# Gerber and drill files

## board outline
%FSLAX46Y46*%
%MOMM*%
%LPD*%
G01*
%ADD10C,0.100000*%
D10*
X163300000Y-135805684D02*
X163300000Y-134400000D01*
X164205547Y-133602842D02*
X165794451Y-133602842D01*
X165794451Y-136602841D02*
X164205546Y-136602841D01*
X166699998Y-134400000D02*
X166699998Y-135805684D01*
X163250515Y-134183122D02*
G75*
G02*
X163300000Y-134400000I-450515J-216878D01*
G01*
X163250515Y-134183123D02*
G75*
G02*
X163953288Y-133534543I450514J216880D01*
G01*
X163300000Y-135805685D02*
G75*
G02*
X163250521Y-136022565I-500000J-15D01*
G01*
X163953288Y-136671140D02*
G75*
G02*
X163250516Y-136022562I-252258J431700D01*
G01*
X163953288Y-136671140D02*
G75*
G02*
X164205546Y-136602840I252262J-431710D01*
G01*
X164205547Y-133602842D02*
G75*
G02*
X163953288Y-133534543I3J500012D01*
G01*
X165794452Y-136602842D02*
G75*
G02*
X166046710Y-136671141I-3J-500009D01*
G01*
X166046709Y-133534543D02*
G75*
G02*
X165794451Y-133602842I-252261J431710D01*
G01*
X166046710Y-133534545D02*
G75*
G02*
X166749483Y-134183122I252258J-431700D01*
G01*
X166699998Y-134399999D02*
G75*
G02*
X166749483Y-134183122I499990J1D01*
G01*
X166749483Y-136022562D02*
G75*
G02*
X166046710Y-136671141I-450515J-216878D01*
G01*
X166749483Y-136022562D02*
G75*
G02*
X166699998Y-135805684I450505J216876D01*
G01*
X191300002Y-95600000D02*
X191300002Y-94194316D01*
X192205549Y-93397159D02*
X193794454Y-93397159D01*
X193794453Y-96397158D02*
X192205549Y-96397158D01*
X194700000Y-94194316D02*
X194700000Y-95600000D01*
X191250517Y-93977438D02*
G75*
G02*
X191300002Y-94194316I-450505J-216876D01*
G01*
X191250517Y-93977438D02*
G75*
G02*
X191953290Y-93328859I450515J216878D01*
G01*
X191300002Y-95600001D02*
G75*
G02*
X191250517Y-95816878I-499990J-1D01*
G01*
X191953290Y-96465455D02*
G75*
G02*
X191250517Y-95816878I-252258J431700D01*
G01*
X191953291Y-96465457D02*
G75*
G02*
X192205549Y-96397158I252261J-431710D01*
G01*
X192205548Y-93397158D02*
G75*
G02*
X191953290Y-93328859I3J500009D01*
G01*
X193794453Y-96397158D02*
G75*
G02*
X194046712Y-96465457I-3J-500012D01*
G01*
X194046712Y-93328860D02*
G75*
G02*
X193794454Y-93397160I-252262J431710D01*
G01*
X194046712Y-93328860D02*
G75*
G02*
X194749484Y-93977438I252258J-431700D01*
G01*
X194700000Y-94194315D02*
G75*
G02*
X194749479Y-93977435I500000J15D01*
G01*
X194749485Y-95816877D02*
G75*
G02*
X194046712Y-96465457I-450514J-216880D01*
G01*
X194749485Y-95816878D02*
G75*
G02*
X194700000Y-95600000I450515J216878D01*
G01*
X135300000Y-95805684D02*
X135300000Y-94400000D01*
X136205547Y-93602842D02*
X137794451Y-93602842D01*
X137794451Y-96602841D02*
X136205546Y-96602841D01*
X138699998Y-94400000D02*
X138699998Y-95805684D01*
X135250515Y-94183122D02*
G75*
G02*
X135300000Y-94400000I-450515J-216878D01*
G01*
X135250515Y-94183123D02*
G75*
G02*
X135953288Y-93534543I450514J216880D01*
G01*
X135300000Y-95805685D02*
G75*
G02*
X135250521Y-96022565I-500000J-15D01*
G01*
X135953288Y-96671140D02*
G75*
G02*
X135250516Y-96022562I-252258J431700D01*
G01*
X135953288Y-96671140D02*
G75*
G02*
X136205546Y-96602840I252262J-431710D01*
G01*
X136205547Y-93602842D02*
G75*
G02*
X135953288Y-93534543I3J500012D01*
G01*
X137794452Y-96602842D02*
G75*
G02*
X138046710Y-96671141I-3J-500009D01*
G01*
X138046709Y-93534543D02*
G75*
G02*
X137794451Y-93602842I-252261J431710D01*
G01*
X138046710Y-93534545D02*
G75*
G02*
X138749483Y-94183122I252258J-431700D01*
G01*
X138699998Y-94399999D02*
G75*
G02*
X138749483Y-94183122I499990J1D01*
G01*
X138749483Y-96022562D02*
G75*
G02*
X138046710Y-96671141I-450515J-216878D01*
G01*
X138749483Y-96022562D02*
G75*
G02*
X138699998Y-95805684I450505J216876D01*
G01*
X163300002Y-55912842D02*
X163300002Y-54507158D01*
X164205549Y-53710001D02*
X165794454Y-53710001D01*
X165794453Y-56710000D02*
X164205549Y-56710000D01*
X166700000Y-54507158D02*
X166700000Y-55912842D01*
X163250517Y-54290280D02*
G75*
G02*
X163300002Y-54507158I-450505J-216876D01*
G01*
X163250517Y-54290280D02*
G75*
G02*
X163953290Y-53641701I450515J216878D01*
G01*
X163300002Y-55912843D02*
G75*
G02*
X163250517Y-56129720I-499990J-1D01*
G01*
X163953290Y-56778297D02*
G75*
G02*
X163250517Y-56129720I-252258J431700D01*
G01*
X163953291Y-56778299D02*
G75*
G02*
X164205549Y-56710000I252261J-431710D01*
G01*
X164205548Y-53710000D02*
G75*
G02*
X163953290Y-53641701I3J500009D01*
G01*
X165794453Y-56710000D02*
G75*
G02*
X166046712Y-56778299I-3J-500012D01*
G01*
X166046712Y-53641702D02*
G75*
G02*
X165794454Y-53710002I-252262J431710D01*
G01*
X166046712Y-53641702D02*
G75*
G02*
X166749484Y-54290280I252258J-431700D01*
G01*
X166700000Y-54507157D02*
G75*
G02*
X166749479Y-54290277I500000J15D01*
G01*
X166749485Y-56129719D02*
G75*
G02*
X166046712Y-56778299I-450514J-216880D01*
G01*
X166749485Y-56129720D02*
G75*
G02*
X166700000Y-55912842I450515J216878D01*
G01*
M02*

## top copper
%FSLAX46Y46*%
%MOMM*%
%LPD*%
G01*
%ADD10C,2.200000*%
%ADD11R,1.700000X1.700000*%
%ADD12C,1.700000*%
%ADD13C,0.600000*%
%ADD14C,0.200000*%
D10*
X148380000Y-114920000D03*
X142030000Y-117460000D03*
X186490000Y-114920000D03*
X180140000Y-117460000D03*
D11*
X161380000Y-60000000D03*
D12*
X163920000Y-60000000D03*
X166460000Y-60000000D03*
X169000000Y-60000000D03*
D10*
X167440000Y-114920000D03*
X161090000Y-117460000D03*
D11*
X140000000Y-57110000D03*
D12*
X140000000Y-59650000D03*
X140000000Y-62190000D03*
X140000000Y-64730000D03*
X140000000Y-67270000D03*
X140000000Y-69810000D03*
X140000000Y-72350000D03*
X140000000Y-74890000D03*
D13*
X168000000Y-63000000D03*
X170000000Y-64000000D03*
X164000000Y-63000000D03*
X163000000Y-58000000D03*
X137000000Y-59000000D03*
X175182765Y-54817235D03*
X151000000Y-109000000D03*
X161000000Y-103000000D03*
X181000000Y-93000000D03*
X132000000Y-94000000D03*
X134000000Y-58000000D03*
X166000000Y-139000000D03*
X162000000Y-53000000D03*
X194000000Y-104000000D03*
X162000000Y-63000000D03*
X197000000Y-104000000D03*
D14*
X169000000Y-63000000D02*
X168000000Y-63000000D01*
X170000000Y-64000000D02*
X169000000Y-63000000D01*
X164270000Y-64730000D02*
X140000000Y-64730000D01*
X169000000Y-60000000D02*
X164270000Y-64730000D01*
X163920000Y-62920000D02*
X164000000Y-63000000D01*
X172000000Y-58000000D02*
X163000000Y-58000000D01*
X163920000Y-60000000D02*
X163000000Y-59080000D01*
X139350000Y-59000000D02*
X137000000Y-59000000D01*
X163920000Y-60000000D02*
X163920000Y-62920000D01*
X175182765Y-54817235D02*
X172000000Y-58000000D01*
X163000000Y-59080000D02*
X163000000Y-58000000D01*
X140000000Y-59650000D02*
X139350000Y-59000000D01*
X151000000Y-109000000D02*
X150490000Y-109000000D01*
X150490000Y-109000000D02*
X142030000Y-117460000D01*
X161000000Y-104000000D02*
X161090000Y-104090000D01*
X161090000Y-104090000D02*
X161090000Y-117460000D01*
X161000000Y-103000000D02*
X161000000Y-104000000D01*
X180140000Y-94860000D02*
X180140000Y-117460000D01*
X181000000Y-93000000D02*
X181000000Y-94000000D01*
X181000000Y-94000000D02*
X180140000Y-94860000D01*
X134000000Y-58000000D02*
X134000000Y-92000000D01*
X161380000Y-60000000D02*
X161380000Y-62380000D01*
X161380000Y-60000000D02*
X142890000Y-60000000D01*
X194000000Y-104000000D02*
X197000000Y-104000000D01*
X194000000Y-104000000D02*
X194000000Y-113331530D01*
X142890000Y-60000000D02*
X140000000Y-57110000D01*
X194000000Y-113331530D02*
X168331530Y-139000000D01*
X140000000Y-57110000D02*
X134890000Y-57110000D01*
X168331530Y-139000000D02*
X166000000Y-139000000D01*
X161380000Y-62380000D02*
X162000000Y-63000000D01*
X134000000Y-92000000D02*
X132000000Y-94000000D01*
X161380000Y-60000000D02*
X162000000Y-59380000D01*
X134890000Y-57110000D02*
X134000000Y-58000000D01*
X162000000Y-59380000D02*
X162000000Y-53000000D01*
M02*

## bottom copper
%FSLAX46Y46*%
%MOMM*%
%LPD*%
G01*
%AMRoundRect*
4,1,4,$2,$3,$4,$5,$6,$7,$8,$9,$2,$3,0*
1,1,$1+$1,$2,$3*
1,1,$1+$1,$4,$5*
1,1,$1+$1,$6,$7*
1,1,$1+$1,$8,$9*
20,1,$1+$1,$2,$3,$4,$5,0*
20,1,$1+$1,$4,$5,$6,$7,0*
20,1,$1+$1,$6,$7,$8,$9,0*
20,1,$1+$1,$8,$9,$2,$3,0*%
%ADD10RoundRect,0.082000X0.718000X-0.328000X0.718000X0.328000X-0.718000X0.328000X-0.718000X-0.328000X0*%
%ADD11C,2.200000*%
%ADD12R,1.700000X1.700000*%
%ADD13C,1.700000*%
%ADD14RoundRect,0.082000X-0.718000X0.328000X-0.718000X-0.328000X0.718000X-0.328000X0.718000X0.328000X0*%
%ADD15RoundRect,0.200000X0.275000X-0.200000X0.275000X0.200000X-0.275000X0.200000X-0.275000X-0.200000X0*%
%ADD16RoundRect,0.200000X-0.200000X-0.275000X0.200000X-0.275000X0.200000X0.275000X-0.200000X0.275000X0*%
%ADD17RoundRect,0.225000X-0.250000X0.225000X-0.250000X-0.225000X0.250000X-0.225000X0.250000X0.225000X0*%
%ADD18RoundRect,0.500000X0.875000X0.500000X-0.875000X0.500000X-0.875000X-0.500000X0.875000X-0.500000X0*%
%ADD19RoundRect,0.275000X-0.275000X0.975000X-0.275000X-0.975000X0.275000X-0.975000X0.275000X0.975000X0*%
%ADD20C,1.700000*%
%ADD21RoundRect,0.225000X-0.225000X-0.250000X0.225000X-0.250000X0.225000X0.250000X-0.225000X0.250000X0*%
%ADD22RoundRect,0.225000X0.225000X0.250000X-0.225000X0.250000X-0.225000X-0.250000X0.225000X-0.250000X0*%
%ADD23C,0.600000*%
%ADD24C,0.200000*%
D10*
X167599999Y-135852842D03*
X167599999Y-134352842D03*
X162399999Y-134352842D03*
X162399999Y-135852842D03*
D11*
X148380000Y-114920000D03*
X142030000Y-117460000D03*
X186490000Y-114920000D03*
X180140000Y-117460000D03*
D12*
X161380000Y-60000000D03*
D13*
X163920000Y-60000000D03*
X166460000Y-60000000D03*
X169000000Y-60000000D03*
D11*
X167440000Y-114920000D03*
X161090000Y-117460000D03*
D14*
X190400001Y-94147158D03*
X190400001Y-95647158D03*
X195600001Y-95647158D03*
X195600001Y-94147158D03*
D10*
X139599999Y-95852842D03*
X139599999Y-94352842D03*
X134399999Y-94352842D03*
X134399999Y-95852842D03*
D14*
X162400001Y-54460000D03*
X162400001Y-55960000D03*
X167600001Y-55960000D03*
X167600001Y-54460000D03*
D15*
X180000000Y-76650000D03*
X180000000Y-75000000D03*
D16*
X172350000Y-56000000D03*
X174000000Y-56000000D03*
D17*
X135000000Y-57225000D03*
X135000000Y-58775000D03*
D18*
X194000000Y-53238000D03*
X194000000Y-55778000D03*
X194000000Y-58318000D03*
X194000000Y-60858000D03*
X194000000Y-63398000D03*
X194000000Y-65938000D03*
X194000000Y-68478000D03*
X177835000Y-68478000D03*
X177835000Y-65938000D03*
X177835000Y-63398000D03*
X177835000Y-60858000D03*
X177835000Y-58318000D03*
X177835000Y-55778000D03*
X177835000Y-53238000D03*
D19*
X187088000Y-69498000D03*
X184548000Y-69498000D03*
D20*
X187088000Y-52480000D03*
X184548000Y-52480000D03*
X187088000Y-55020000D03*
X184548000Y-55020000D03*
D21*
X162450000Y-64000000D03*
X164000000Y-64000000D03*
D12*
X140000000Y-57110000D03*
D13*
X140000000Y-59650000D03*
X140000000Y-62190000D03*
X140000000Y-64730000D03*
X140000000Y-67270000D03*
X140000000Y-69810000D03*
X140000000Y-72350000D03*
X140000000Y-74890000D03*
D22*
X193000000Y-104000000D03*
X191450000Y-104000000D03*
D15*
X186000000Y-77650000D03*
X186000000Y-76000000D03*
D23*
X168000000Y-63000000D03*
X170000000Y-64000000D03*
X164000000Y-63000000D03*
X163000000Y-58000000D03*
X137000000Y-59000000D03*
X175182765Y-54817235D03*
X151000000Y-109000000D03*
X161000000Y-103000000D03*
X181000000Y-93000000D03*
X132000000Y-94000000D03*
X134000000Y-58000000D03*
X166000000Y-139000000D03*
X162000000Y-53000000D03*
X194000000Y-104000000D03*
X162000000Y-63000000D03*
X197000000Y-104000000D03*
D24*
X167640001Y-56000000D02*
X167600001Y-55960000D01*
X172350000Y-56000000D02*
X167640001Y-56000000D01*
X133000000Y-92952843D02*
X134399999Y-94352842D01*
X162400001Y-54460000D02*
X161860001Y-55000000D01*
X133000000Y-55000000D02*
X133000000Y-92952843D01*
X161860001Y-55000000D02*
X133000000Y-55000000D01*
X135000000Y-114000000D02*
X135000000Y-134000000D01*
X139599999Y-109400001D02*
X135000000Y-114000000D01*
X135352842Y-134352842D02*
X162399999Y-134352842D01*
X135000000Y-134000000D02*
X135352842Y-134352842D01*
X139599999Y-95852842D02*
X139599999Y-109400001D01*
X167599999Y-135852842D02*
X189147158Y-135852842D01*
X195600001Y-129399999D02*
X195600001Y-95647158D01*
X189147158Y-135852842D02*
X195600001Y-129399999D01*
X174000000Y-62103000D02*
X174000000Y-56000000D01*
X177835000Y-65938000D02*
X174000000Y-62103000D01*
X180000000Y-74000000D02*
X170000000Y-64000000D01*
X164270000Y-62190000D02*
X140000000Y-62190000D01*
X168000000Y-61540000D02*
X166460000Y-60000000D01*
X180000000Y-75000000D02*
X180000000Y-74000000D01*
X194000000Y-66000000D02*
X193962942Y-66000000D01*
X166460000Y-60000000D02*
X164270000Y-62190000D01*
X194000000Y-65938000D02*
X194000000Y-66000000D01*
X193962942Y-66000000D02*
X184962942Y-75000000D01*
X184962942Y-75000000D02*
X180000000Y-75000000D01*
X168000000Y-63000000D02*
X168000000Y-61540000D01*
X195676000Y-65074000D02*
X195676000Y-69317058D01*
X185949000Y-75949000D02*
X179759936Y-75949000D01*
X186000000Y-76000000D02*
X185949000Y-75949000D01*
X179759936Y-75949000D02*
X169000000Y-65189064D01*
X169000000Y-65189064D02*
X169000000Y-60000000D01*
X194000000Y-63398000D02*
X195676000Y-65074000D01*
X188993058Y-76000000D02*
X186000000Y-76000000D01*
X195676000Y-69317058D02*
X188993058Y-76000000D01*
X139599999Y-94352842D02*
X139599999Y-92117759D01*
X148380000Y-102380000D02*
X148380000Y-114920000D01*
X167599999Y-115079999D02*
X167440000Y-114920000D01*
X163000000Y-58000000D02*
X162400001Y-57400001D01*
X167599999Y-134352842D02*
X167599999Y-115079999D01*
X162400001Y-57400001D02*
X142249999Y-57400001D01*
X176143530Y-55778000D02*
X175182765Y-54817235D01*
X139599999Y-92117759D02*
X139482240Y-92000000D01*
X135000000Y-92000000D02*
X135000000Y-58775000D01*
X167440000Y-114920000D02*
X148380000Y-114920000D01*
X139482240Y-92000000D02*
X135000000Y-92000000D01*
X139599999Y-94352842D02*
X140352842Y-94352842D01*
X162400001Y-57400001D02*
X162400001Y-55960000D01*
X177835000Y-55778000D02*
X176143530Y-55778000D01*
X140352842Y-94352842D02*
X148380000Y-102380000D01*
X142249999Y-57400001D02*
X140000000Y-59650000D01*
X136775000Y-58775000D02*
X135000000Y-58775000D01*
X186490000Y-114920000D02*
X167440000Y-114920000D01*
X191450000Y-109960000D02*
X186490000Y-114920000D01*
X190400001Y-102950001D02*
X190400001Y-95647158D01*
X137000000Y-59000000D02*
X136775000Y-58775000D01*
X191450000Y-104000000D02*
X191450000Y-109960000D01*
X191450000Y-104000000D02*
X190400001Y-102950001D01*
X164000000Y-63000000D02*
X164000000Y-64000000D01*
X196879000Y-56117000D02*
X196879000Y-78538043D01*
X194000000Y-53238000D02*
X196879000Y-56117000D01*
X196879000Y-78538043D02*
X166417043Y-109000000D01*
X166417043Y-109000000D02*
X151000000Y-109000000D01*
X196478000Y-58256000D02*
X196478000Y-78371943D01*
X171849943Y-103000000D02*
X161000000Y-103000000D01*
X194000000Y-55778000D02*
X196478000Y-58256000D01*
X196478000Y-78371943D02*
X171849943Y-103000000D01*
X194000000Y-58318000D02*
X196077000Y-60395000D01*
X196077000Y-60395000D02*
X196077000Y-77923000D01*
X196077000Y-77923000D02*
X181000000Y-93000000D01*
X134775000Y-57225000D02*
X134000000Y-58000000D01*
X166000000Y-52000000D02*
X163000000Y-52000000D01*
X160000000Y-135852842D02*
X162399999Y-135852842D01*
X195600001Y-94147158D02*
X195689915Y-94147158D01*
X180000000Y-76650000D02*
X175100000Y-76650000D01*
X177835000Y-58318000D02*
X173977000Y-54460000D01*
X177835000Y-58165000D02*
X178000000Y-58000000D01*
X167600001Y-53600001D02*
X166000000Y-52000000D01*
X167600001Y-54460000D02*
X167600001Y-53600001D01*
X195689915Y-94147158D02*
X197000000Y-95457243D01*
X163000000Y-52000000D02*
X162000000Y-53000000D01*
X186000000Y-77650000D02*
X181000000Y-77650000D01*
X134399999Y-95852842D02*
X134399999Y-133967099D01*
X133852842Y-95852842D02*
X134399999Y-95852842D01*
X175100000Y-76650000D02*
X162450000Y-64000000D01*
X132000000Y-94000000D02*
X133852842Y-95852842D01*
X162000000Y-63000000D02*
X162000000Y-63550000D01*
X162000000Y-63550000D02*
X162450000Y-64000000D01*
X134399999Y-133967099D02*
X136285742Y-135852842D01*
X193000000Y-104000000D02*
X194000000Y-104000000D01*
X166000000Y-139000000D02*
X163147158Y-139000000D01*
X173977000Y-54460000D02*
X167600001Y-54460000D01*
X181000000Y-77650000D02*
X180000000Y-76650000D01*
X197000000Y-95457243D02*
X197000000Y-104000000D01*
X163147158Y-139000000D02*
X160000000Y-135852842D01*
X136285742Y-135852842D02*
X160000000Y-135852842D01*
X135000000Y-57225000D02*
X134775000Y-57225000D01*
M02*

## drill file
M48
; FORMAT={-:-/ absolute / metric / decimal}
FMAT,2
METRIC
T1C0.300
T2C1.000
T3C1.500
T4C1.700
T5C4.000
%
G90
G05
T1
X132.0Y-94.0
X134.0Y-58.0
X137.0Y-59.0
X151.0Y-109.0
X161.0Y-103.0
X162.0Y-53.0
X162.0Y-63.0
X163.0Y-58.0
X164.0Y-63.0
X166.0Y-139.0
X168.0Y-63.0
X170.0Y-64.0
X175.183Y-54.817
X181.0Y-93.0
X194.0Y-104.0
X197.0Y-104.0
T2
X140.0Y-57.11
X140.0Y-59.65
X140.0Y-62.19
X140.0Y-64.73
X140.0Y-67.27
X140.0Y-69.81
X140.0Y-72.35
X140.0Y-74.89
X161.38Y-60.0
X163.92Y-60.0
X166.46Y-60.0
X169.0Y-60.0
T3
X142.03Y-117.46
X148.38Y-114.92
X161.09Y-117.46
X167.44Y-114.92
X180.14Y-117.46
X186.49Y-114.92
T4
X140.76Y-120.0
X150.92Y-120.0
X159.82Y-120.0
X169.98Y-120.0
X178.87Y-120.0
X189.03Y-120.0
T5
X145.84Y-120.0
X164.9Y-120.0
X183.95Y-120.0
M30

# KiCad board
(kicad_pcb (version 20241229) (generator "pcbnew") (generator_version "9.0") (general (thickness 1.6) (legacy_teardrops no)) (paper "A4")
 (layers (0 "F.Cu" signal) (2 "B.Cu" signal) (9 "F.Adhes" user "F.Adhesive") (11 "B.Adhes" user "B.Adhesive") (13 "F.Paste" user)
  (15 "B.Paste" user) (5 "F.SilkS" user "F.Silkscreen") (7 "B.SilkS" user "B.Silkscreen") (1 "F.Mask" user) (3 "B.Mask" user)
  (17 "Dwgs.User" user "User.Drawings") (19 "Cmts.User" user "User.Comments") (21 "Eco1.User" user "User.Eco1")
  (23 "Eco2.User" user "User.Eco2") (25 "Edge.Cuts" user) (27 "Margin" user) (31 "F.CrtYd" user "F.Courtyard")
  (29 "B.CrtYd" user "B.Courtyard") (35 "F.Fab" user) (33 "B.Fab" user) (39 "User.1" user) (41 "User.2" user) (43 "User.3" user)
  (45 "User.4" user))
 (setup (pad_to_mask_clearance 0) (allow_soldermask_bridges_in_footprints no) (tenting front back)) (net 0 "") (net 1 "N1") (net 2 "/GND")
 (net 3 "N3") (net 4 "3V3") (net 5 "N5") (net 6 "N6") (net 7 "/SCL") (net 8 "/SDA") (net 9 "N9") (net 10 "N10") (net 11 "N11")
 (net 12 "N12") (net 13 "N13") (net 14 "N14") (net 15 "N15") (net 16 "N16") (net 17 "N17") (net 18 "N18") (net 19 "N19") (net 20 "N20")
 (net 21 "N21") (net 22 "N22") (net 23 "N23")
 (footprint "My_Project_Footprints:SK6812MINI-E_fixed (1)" (layer "F.Cu") (at 165 135 180)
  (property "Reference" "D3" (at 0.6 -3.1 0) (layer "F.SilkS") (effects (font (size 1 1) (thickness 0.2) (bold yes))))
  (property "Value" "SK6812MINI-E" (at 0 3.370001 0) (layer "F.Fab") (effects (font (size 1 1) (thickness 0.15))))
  (fp_line (start 1.7 -0.805684) (end 1.7 0.6) (stroke (width 0.1) (type solid)) (layer "Edge.Cuts"))
  (fp_line (start 0.794453 1.397158) (end -0.794451 1.397158) (stroke (width 0.1) (type solid)) (layer "Edge.Cuts"))
  (fp_line (start -0.794451 -1.602841) (end 0.794454 -1.602841) (stroke (width 0.1) (type solid)) (layer "Edge.Cuts"))
  (fp_line (start -1.699998 0.6) (end -1.699998 -0.805684) (stroke (width 0.1) (type solid)) (layer "Edge.Cuts"))
  (fp_arc (start 1.749485 0.816878) (mid 1.712528 0.711226) (end 1.7 0.6) (stroke (width 0.1) (type solid)) (layer "Edge.Cuts"))
  (fp_arc (start 1.749485 0.816877) (mid 1.638073 1.401193) (end 1.046712 1.465457) (stroke (width 0.1) (type solid)) (layer "Edge.Cuts"))
  (fp_arc (start 1.7 -0.805685) (mid 1.712528 -0.91691) (end 1.749485 -1.022562) (stroke (width 0.1) (type solid)) (layer "Edge.Cuts"))
  (fp_arc (start 1.046712 -1.67114) (mid 1.638072 -1.606876) (end 1.749485 -1.022562) (stroke (width 0.1) (type solid)) (layer "Edge.Cuts"))
  (fp_arc (start 1.046712 -1.67114) (mid 0.925124 -1.620218) (end 0.794454 -1.602841) (stroke (width 0.1) (type solid)) (layer "Edge.Cuts"))
  (fp_arc (start 0.794453 1.397158) (mid 0.925124 1.414535) (end 1.046712 1.465457) (stroke (width 0.1) (type solid)) (layer "Edge.Cuts"))
  (fp_arc (start -0.794452 -1.602842) (mid -0.925122 -1.620219) (end -1.04671 -1.671141) (stroke (width 0.1) (type solid))
   (layer "Edge.Cuts"))
  (fp_arc (start -1.046709 1.465457) (mid -0.925121 1.414535) (end -0.794451 1.397158) (stroke (width 0.1) (type solid)) (layer "Edge.Cuts"))
  (fp_arc (start -1.04671 1.465455) (mid -1.638069 1.401192) (end -1.749483 0.816878) (stroke (width 0.1) (type solid)) (layer "Edge.Cuts"))
  (fp_arc (start -1.699998 0.600001) (mid -1.712526 0.711226) (end -1.749483 0.816878) (stroke (width 0.1) (type solid)) (layer "Edge.Cuts"))
  (fp_arc (start -1.749483 -1.022562) (mid -1.63807 -1.606877) (end -1.04671 -1.671141) (stroke (width 0.1) (type solid))
   (layer "Edge.Cuts"))
  (fp_arc (start -1.749483 -1.022562) (mid -1.712526 -0.91691) (end -1.699998 -0.805684) (stroke (width 0.1) (type solid))
   (layer "Edge.Cuts"))
  (pad "1" smd roundrect (at -2.599999 -0.852842 90) (size 0.82 1.6) (layers "B.Cu" "B.Mask" "B.Paste") (roundrect_rratio 0.1) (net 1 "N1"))
  (pad "2" smd roundrect (at -2.599999 0.647158 90) (size 0.82 1.6) (layers "B.Cu" "B.Mask" "B.Paste") (roundrect_rratio 0.1) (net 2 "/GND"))
  (pad "3" smd roundrect (at 2.600001 0.647158 90) (size 0.82 1.6) (layers "B.Cu" "B.Mask" "B.Paste") (roundrect_rratio 0.1) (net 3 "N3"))
  (pad "4" smd roundrect (at 2.600001 -0.852842 90) (size 0.82 1.6) (layers "B.Cu" "B.Mask" "B.Paste") (roundrect_rratio 0.1) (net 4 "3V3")))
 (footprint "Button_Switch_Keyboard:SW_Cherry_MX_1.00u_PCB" (layer "F.Cu") (at 148.38 114.92)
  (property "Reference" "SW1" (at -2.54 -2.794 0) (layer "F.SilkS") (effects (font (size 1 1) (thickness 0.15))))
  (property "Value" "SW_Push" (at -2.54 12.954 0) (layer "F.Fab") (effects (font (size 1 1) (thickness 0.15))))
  (pad "" np_thru_hole circle (at -7.62 5.08) (size 1.7 1.7) (drill 1.7) (layers "*.Cu" "*.Mask"))
  (pad "" np_thru_hole circle (at -2.54 5.08) (size 4 4) (drill 4) (layers "*.Cu" "*.Mask"))
  (pad "" np_thru_hole circle (at 2.54 5.08) (size 1.7 1.7) (drill 1.7) (layers "*.Cu" "*.Mask"))
  (pad "1" thru_hole circle (at 0 0) (size 2.2 2.2) (drill 1.5) (layers "*.Cu" "*.Mask") (remove_unused_layers no) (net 2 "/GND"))
  (pad "2" thru_hole circle (at -6.35 2.54) (size 2.2 2.2) (drill 1.5) (layers "*.Cu" "*.Mask") (remove_unused_layers no) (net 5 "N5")))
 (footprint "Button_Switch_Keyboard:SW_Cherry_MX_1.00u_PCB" (layer "F.Cu") (at 186.49 114.92)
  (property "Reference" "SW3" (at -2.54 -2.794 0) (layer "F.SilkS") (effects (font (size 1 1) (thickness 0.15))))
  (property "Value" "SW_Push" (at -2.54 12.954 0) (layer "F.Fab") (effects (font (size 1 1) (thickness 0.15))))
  (pad "" np_thru_hole circle (at -7.62 5.08) (size 1.7 1.7) (drill 1.7) (layers "*.Cu" "*.Mask"))
  (pad "" np_thru_hole circle (at -2.54 5.08) (size 4 4) (drill 4) (layers "*.Cu" "*.Mask"))
  (pad "" np_thru_hole circle (at 2.54 5.08) (size 1.7 1.7) (drill 1.7) (layers "*.Cu" "*.Mask"))
  (pad "1" thru_hole circle (at 0 0) (size 2.2 2.2) (drill 1.5) (layers "*.Cu" "*.Mask") (remove_unused_layers no) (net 2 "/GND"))
  (pad "2" thru_hole circle (at -6.35 2.54) (size 2.2 2.2) (drill 1.5) (layers "*.Cu" "*.Mask") (remove_unused_layers no) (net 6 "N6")))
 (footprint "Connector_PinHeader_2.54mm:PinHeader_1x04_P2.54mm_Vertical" (layer "F.Cu") (at 161.38 60 90)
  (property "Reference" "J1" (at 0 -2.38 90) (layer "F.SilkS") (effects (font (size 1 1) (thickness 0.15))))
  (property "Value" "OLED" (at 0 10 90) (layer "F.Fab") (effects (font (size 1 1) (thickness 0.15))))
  (pad "1" thru_hole rect (at 0 0 90) (size 1.7 1.7) (drill 1) (layers "*.Cu" "*.Mask") (remove_unused_layers no) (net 4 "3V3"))
  (pad "2" thru_hole circle (at 0 2.54 90) (size 1.7 1.7) (drill 1) (layers "*.Cu" "*.Mask") (remove_unused_layers no) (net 2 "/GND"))
  (pad "3" thru_hole circle (at 0 5.08 90) (size 1.7 1.7) (drill 1) (layers "*.Cu" "*.Mask") (remove_unused_layers no) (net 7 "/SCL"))
  (pad "4" thru_hole circle (at 0 7.62 90) (size 1.7 1.7) (drill 1) (layers "*.Cu" "*.Mask") (remove_unused_layers no) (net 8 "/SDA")))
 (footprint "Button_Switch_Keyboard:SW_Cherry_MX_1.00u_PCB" (layer "F.Cu") (at 167.44 114.92)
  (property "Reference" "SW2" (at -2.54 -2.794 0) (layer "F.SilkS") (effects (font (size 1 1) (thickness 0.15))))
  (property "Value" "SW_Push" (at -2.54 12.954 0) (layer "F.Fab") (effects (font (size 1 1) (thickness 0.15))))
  (pad "" np_thru_hole circle (at -7.62 5.08) (size 1.7 1.7) (drill 1.7) (layers "*.Cu" "*.Mask"))
  (pad "" np_thru_hole circle (at -2.54 5.08) (size 4 4) (drill 4) (layers "*.Cu" "*.Mask"))
  (pad "" np_thru_hole circle (at 2.54 5.08) (size 1.7 1.7) (drill 1.7) (layers "*.Cu" "*.Mask"))
  (pad "1" thru_hole circle (at 0 0) (size 2.2 2.2) (drill 1.5) (layers "*.Cu" "*.Mask") (remove_unused_layers no) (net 2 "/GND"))
  (pad "2" thru_hole circle (at -6.35 2.54) (size 2.2 2.2) (drill 1.5) (layers "*.Cu" "*.Mask") (remove_unused_layers no) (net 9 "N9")))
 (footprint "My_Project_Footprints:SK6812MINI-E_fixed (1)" (layer "F.Cu") (at 193 95)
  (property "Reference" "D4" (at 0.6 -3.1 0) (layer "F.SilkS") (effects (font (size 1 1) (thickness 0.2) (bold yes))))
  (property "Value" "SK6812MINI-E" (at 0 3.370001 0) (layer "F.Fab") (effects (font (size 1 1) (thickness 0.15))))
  (fp_line (start -1.699998 0.6) (end -1.699998 -0.805684) (stroke (width 0.1) (type solid)) (layer "Edge.Cuts"))
  (fp_line (start -0.794451 -1.602841) (end 0.794454 -1.602841) (stroke (width 0.1) (type solid)) (layer "Edge.Cuts"))
  (fp_line (start 0.794453 1.397158) (end -0.794451 1.397158) (stroke (width 0.1) (type solid)) (layer "Edge.Cuts"))
  (fp_line (start 1.7 -0.805684) (end 1.7 0.6) (stroke (width 0.1) (type solid)) (layer "Edge.Cuts"))
  (fp_arc (start -1.749483 -1.022562) (mid -1.712526 -0.91691) (end -1.699998 -0.805684) (stroke (width 0.1) (type solid))
   (layer "Edge.Cuts"))
  (fp_arc (start -1.749483 -1.022562) (mid -1.63807 -1.606877) (end -1.04671 -1.671141) (stroke (width 0.1) (type solid))
   (layer "Edge.Cuts"))
  (fp_arc (start -1.699998 0.600001) (mid -1.712526 0.711226) (end -1.749483 0.816878) (stroke (width 0.1) (type solid)) (layer "Edge.Cuts"))
  (fp_arc (start -1.04671 1.465455) (mid -1.638069 1.401192) (end -1.749483 0.816878) (stroke (width 0.1) (type solid)) (layer "Edge.Cuts"))
  (fp_arc (start -1.046709 1.465457) (mid -0.925121 1.414535) (end -0.794451 1.397158) (stroke (width 0.1) (type solid)) (layer "Edge.Cuts"))
  (fp_arc (start -0.794452 -1.602842) (mid -0.925122 -1.620219) (end -1.04671 -1.671141) (stroke (width 0.1) (type solid))
   (layer "Edge.Cuts"))
  (fp_arc (start 0.794453 1.397158) (mid 0.925124 1.414535) (end 1.046712 1.465457) (stroke (width 0.1) (type solid)) (layer "Edge.Cuts"))
  (fp_arc (start 1.046712 -1.67114) (mid 0.925124 -1.620218) (end 0.794454 -1.602841) (stroke (width 0.1) (type solid)) (layer "Edge.Cuts"))
  (fp_arc (start 1.046712 -1.67114) (mid 1.638072 -1.606876) (end 1.749485 -1.022562) (stroke (width 0.1) (type solid)) (layer "Edge.Cuts"))
  (fp_arc (start 1.7 -0.805685) (mid 1.712528 -0.91691) (end 1.749485 -1.022562) (stroke (width 0.1) (type solid)) (layer "Edge.Cuts"))
  (fp_arc (start 1.749485 0.816877) (mid 1.638073 1.401193) (end 1.046712 1.465457) (stroke (width 0.1) (type solid)) (layer "Edge.Cuts"))
  (fp_arc (start 1.749485 0.816878) (mid 1.712528 0.711226) (end 1.7 0.6) (stroke (width 0.1) (type solid)) (layer "Edge.Cuts"))
  (pad "1" smd roundrect (at -2.599999 -0.852842 270) (size 0.82 1.6) (layers "B.Cu" "B.Mask" "B.Paste") (roundrect_rratio 0.1)
   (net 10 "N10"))
  (pad "2" smd roundrect (at -2.599999 0.647158 270) (size 0.82 1.6) (layers "B.Cu" "B.Mask" "B.Paste") (roundrect_rratio 0.1)
   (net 2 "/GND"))
  (pad "3" smd roundrect (at 2.600001 0.647158 270) (size 0.82 1.6) (layers "B.Cu" "B.Mask" "B.Paste") (roundrect_rratio 0.1) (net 1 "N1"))
  (pad "4" smd roundrect (at 2.600001 -0.852842 270) (size 0.82 1.6) (layers "B.Cu" "B.Mask" "B.Paste") (roundrect_rratio 0.1) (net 4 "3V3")))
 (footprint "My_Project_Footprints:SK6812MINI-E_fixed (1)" (layer "F.Cu") (at 137 95 180)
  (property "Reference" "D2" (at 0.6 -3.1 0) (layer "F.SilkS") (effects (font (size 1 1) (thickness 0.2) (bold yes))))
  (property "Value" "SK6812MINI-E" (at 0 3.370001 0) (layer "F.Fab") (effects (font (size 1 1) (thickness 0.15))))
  (fp_line (start 1.7 -0.805684) (end 1.7 0.6) (stroke (width 0.1) (type solid)) (layer "Edge.Cuts"))
  (fp_line (start 0.794453 1.397158) (end -0.794451 1.397158) (stroke (width 0.1) (type solid)) (layer "Edge.Cuts"))
  (fp_line (start -0.794451 -1.602841) (end 0.794454 -1.602841) (stroke (width 0.1) (type solid)) (layer "Edge.Cuts"))
  (fp_line (start -1.699998 0.6) (end -1.699998 -0.805684) (stroke (width 0.1) (type solid)) (layer "Edge.Cuts"))
  (fp_arc (start 1.749485 0.816878) (mid 1.712528 0.711226) (end 1.7 0.6) (stroke (width 0.1) (type solid)) (layer "Edge.Cuts"))
  (fp_arc (start 1.749485 0.816877) (mid 1.638073 1.401193) (end 1.046712 1.465457) (stroke (width 0.1) (type solid)) (layer "Edge.Cuts"))
  (fp_arc (start 1.7 -0.805685) (mid 1.712528 -0.91691) (end 1.749485 -1.022562) (stroke (width 0.1) (type solid)) (layer "Edge.Cuts"))
  (fp_arc (start 1.046712 -1.67114) (mid 1.638072 -1.606876) (end 1.749485 -1.022562) (stroke (width 0.1) (type solid)) (layer "Edge.Cuts"))
  (fp_arc (start 1.046712 -1.67114) (mid 0.925124 -1.620218) (end 0.794454 -1.602841) (stroke (width 0.1) (type solid)) (layer "Edge.Cuts"))
  (fp_arc (start 0.794453 1.397158) (mid 0.925124 1.414535) (end 1.046712 1.465457) (stroke (width 0.1) (type solid)) (layer "Edge.Cuts"))
  (fp_arc (start -0.794452 -1.602842) (mid -0.925122 -1.620219) (end -1.04671 -1.671141) (stroke (width 0.1) (type solid))
   (layer "Edge.Cuts"))
  (fp_arc (start -1.046709 1.465457) (mid -0.925121 1.414535) (end -0.794451 1.397158) (stroke (width 0.1) (type solid)) (layer "Edge.Cuts"))
  (fp_arc (start -1.04671 1.465455) (mid -1.638069 1.401192) (end -1.749483 0.816878) (stroke (width 0.1) (type solid)) (layer "Edge.Cuts"))
  (fp_arc (start -1.699998 0.600001) (mid -1.712526 0.711226) (end -1.749483 0.816878) (stroke (width 0.1) (type solid)) (layer "Edge.Cuts"))
  (fp_arc (start -1.749483 -1.022562) (mid -1.63807 -1.606877) (end -1.04671 -1.671141) (stroke (width 0.1) (type solid))
   (layer "Edge.Cuts"))
  (fp_arc (start -1.749483 -1.022562) (mid -1.712526 -0.91691) (end -1.699998 -0.805684) (stroke (width 0.1) (type solid))
   (layer "Edge.Cuts"))
  (pad "1" smd roundrect (at -2.599999 -0.852842 90) (size 0.82 1.6) (layers "B.Cu" "B.Mask" "B.Paste") (roundrect_rratio 0.1) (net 3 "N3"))
  (pad "2" smd roundrect (at -2.599999 0.647158 90) (size 0.82 1.6) (layers "B.Cu" "B.Mask" "B.Paste") (roundrect_rratio 0.1) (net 2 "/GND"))
  (pad "3" smd roundrect (at 2.600001 0.647158 90) (size 0.82 1.6) (layers "B.Cu" "B.Mask" "B.Paste") (roundrect_rratio 0.1) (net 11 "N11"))
  (pad "4" smd roundrect (at 2.600001 -0.852842 90) (size 0.82 1.6) (layers "B.Cu" "B.Mask" "B.Paste") (roundrect_rratio 0.1) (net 4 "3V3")))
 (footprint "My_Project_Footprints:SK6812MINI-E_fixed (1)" (layer "F.Cu") (at 165 55.312842)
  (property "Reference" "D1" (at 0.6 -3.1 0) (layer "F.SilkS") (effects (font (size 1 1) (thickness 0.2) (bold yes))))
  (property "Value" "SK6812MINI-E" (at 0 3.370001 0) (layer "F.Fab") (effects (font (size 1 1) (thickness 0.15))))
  (fp_line (start -1.699998 0.6) (end -1.699998 -0.805684) (stroke (width 0.1) (type solid)) (layer "Edge.Cuts"))
  (fp_line (start -0.794451 -1.602841) (end 0.794454 -1.602841) (stroke (width 0.1) (type solid)) (layer "Edge.Cuts"))
  (fp_line (start 0.794453 1.397158) (end -0.794451 1.397158) (stroke (width 0.1) (type solid)) (layer "Edge.Cuts"))
  (fp_line (start 1.7 -0.805684) (end 1.7 0.6) (stroke (width 0.1) (type solid)) (layer "Edge.Cuts"))
  (fp_arc (start -1.749483 -1.022562) (mid -1.712526 -0.91691) (end -1.699998 -0.805684) (stroke (width 0.1) (type solid))
   (layer "Edge.Cuts"))
  (fp_arc (start -1.749483 -1.022562) (mid -1.63807 -1.606877) (end -1.04671 -1.671141) (stroke (width 0.1) (type solid))
   (layer "Edge.Cuts"))
  (fp_arc (start -1.699998 0.600001) (mid -1.712526 0.711226) (end -1.749483 0.816878) (stroke (width 0.1) (type solid)) (layer "Edge.Cuts"))
  (fp_arc (start -1.04671 1.465455) (mid -1.638069 1.401192) (end -1.749483 0.816878) (stroke (width 0.1) (type solid)) (layer "Edge.Cuts"))
  (fp_arc (start -1.046709 1.465457) (mid -0.925121 1.414535) (end -0.794451 1.397158) (stroke (width 0.1) (type solid)) (layer "Edge.Cuts"))
  (fp_arc (start -0.794452 -1.602842) (mid -0.925122 -1.620219) (end -1.04671 -1.671141) (stroke (width 0.1) (type solid))
   (layer "Edge.Cuts"))
  (fp_arc (start 0.794453 1.397158) (mid 0.925124 1.414535) (end 1.046712 1.465457) (stroke (width 0.1) (type solid)) (layer "Edge.Cuts"))
  (fp_arc (start 1.046712 -1.67114) (mid 0.925124 -1.620218) (end 0.794454 -1.602841) (stroke (width 0.1) (type solid)) (layer "Edge.Cuts"))
  (fp_arc (start 1.046712 -1.67114) (mid 1.638072 -1.606876) (end 1.749485 -1.022562) (stroke (width 0.1) (type solid)) (layer "Edge.Cuts"))
  (fp_arc (start 1.7 -0.805685) (mid 1.712528 -0.91691) (end 1.749485 -1.022562) (stroke (width 0.1) (type solid)) (layer "Edge.Cuts"))
  (fp_arc (start 1.749485 0.816877) (mid 1.638073 1.401193) (end 1.046712 1.465457) (stroke (width 0.1) (type solid)) (layer "Edge.Cuts"))
  (fp_arc (start 1.749485 0.816878) (mid 1.712528 0.711226) (end 1.7 0.6) (stroke (width 0.1) (type solid)) (layer "Edge.Cuts"))
  (pad "1" smd roundrect (at -2.599999 -0.852842 270) (size 0.82 1.6) (layers "B.Cu" "B.Mask" "B.Paste") (roundrect_rratio 0.1)
   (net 11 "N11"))
  (pad "2" smd roundrect (at -2.599999 0.647158 270) (size 0.82 1.6) (layers "B.Cu" "B.Mask" "B.Paste") (roundrect_rratio 0.1)
   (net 2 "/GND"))
  (pad "3" smd roundrect (at 2.600001 0.647158 270) (size 0.82 1.6) (layers "B.Cu" "B.Mask" "B.Paste") (roundrect_rratio 0.1) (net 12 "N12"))
  (pad "4" smd roundrect (at 2.600001 -0.852842 270) (size 0.82 1.6) (layers "B.Cu" "B.Mask" "B.Paste") (roundrect_rratio 0.1) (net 4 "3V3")))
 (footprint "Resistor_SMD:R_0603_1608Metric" (layer "B.Cu") (at 180 75.825 90)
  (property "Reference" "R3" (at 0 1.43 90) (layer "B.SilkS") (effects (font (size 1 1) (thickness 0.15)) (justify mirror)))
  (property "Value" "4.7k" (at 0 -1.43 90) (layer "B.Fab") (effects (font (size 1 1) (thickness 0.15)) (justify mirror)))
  (pad "1" smd roundrect (at -0.825 0 90) (size 0.8 0.95) (layers "B.Cu" "B.Mask" "B.Paste") (roundrect_rratio 0.25) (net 4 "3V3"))
  (pad "2" smd roundrect (at 0.825 0 90) (size 0.8 0.95) (layers "B.Cu" "B.Mask" "B.Paste") (roundrect_rratio 0.25) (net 7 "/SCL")))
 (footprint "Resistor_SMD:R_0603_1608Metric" (layer "B.Cu") (at 173.175 56)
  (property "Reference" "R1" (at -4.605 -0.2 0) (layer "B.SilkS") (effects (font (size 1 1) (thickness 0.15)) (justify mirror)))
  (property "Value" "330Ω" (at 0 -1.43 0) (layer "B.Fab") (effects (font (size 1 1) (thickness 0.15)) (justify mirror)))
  (pad "1" smd roundrect (at -0.825 0) (size 0.8 0.95) (layers "B.Cu" "B.Mask" "B.Paste") (roundrect_rratio 0.25) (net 12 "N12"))
  (pad "2" smd roundrect (at 0.825 0) (size 0.8 0.95) (layers "B.Cu" "B.Mask" "B.Paste") (roundrect_rratio 0.25) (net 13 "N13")))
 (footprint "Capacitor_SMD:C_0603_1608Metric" (layer "B.Cu") (at 135 58 -90)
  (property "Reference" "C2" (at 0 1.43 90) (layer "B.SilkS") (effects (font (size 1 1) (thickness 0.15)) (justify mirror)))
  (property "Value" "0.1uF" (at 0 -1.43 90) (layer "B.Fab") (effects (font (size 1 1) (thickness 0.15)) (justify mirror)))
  (pad "1" smd roundrect (at -0.775 0 270) (size 0.9 0.95) (layers "B.Cu" "B.Mask" "B.Paste") (roundrect_rratio 0.25) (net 4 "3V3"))
  (pad "2" smd roundrect (at 0.775 0 270) (size 0.9 0.95) (layers "B.Cu" "B.Mask" "B.Paste") (roundrect_rratio 0.25) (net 2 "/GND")))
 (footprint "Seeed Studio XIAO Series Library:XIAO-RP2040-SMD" (layer "B.Cu") (at 186 60.858 180)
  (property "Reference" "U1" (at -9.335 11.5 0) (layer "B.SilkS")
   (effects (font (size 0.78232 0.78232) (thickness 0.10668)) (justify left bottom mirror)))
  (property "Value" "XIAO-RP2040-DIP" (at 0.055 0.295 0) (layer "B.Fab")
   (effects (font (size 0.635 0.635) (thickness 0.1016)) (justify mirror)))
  (pad "1" smd roundrect (at -8 7.62 180) (size 2.75 2) (layers "B.Cu" "B.Mask" "B.Paste") (roundrect_rratio 0.25) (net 5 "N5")
   (solder_mask_margin 0.0508) (thermal_bridge_angle 45))
  (pad "2" smd roundrect (at -8 5.08 180) (size 2.75 2) (layers "B.Cu" "B.Mask" "B.Paste") (roundrect_rratio 0.25) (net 9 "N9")
   (solder_mask_margin 0.0508) (thermal_bridge_angle 45))
  (pad "3" smd roundrect (at -8 2.54 180) (size 2.75 2) (layers "B.Cu" "B.Mask" "B.Paste") (roundrect_rratio 0.25) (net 6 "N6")
   (solder_mask_margin 0.0508) (thermal_bridge_angle 45))
  (pad "4" smd roundrect (at -8 0 180) (size 2.75 2) (layers "B.Cu" "B.Mask" "B.Paste") (roundrect_rratio 0.25) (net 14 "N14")
   (solder_mask_margin 0.0508) (thermal_bridge_angle 45))
  (pad "5" smd roundrect (at -8 -2.54 180) (size 2.75 2) (layers "B.Cu" "B.Mask" "B.Paste") (roundrect_rratio 0.25) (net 8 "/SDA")
   (solder_mask_margin 0.0508) (thermal_bridge_angle 45))
  (pad "6" smd roundrect (at -8 -5.08 180) (size 2.75 2) (layers "B.Cu" "B.Mask" "B.Paste") (roundrect_rratio 0.25) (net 7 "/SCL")
   (solder_mask_margin 0.0508) (thermal_bridge_angle 45))
  (pad "7" smd roundrect (at -8 -7.62 180) (size 2.75 2) (layers "B.Cu" "B.Mask" "B.Paste") (roundrect_rratio 0.25) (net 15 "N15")
   (solder_mask_margin 0.0508) (thermal_bridge_angle 45))
  (pad "8" smd roundrect (at 8.165 -7.62 180) (size 2.75 2) (layers "B.Cu" "B.Mask" "B.Paste") (roundrect_rratio 0.25) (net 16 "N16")
   (solder_mask_margin 0.0508) (thermal_bridge_angle 45))
  (pad "9" smd roundrect (at 8.165 -5.08 180) (size 2.75 2) (layers "B.Cu" "B.Mask" "B.Paste") (roundrect_rratio 0.25) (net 13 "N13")
   (solder_mask_margin 0.0508) (thermal_bridge_angle 45))
  (pad "10" smd roundrect (at 8.165 -2.54 180) (size 2.75 2) (layers "B.Cu" "B.Mask" "B.Paste") (roundrect_rratio 0.25) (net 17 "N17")
   (solder_mask_margin 0.0508) (thermal_bridge_angle 45))
  (pad "11" smd roundrect (at 8.165 0 180) (size 2.75 2) (layers "B.Cu" "B.Mask" "B.Paste") (roundrect_rratio 0.25) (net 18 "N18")
   (solder_mask_margin 0.0508) (thermal_bridge_angle 45))
  (pad "12" smd roundrect (at 8.165 2.54 180) (size 2.75 2) (layers "B.Cu" "B.Mask" "B.Paste") (roundrect_rratio 0.25) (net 4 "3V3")
   (solder_mask_margin 0.0508) (thermal_bridge_angle 45))
  (pad "13" smd roundrect (at 8.165 5.08 180) (size 2.75 2) (layers "B.Cu" "B.Mask" "B.Paste") (roundrect_rratio 0.25) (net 2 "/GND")
   (solder_mask_margin 0.0508) (thermal_bridge_angle 45))
  (pad "14" smd roundrect (at 8.165 7.62 180) (size 2.75 2) (layers "B.Cu" "B.Mask" "B.Paste") (roundrect_rratio 0.25) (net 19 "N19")
   (solder_mask_margin 0.0508) (thermal_bridge_angle 45))
  (pad "15" smd roundrect (at -1.088 -8.64 270) (size 2.5 1.1) (layers "B.Cu" "B.Mask" "B.Paste") (roundrect_rratio 0.25)
   (thermal_bridge_angle 45))
  (pad "16" smd roundrect (at 1.452 -8.64 270) (size 2.5 1.1) (layers "B.Cu" "B.Mask" "B.Paste") (roundrect_rratio 0.25)
   (thermal_bridge_angle 45))
  (pad "17" smd circle (at -1.088 8.378 180) (size 1.7 1.7) (layers "B.Cu" "B.Mask" "B.Paste"))
  (pad "18" smd circle (at 1.452 8.378 180) (size 1.7 1.7) (layers "B.Cu" "B.Mask" "B.Paste"))
  (pad "19" smd circle (at -1.088 5.838 180) (size 1.7 1.7) (layers "B.Cu" "B.Mask" "B.Paste"))
  (pad "20" smd circle (at 1.452 5.838 180) (size 1.7 1.7) (layers "B.Cu" "B.Mask" "B.Paste")))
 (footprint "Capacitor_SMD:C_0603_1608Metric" (layer "B.Cu") (at 163.225 64)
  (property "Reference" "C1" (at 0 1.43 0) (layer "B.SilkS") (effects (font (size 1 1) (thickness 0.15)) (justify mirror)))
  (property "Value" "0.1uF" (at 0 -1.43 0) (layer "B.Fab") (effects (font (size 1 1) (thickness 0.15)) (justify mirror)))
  (pad "1" smd roundrect (at -0.775 0) (size 0.9 0.95) (layers "B.Cu" "B.Mask" "B.Paste") (roundrect_rratio 0.25) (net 4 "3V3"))
  (pad "2" smd roundrect (at 0.775 0) (size 0.9 0.95) (layers "B.Cu" "B.Mask" "B.Paste") (roundrect_rratio 0.25) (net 2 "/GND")))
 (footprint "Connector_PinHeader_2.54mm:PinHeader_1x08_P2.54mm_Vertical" (layer "B.Cu") (at 140 57.11 180)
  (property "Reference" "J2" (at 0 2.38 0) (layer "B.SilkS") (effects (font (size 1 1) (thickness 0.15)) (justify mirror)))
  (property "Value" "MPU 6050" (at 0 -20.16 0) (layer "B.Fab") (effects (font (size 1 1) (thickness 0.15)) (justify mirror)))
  (pad "1" thru_hole rect (at 0 0 180) (size 1.7 1.7) (drill 1) (layers "*.Cu" "*.Mask") (remove_unused_layers no) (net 4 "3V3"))
  (pad "2" thru_hole circle (at 0 -2.54 180) (size 1.7 1.7) (drill 1) (layers "*.Cu" "*.Mask") (remove_unused_layers no) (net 2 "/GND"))
  (pad "3" thru_hole circle (at 0 -5.08 180) (size 1.7 1.7) (drill 1) (layers "*.Cu" "*.Mask") (remove_unused_layers no) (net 7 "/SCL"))
  (pad "4" thru_hole circle (at 0 -7.62 180) (size 1.7 1.7) (drill 1) (layers "*.Cu" "*.Mask") (remove_unused_layers no) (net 8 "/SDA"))
  (pad "5" thru_hole circle (at 0 -10.16 180) (size 1.7 1.7) (drill 1) (layers "*.Cu" "*.Mask") (remove_unused_layers no) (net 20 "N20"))
  (pad "6" thru_hole circle (at 0 -12.7 180) (size 1.7 1.7) (drill 1) (layers "*.Cu" "*.Mask") (remove_unused_layers no) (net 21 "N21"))
  (pad "7" thru_hole circle (at 0 -15.24 180) (size 1.7 1.7) (drill 1) (layers "*.Cu" "*.Mask") (remove_unused_layers no) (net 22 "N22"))
  (pad "8" thru_hole circle (at 0 -17.78 180) (size 1.7 1.7) (drill 1) (layers "*.Cu" "*.Mask") (remove_unused_layers no) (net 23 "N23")))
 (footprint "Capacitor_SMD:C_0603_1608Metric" (layer "B.Cu") (at 192.225 104 180)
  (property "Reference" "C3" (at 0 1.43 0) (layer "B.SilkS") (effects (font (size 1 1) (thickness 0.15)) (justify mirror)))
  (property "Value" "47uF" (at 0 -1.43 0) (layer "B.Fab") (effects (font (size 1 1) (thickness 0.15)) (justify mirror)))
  (pad "1" smd roundrect (at -0.775 0 180) (size 0.9 0.95) (layers "B.Cu" "B.Mask" "B.Paste") (roundrect_rratio 0.25) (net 4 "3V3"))
  (pad "2" smd roundrect (at 0.775 0 180) (size 0.9 0.95) (layers "B.Cu" "B.Mask" "B.Paste") (roundrect_rratio 0.25) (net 2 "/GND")))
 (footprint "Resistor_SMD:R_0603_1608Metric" (layer "B.Cu") (at 186 76.825 90)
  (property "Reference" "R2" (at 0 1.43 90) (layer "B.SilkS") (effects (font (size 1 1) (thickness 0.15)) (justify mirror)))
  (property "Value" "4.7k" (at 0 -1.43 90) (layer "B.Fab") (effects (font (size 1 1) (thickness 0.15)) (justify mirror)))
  (pad "1" smd roundrect (at -0.825 0 90) (size 0.8 0.95) (layers "B.Cu" "B.Mask" "B.Paste") (roundrect_rratio 0.25) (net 4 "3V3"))
  (pad "2" smd roundrect (at 0.825 0 90) (size 0.8 0.95) (layers "B.Cu" "B.Mask" "B.Paste") (roundrect_rratio 0.25) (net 8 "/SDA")))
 (segment (start 167.640001 56) (end 167.600001 55.96) (width 0.2) (layer "B.Cu") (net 12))
 (segment (start 172.35 56) (end 167.640001 56) (width 0.2) (layer "B.Cu") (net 12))
 (segment (start 133 92.952843) (end 134.399999 94.352842) (width 0.2) (layer "B.Cu") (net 11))
 (segment (start 162.400001 54.46) (end 161.860001 55) (width 0.2) (layer "B.Cu") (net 11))
 (segment (start 133 55) (end 133 92.952843) (width 0.2) (layer "B.Cu") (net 11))
 (segment (start 161.860001 55) (end 133 55) (width 0.2) (layer "B.Cu") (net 11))
 (segment (start 135 114) (end 135 134) (width 0.2) (layer "B.Cu") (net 3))
 (segment (start 139.599999 109.400001) (end 135 114) (width 0.2) (layer "B.Cu") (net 3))
 (segment (start 135.352842 134.352842) (end 162.399999 134.352842) (width 0.2) (layer "B.Cu") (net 3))
 (segment (start 135 134) (end 135.352842 134.352842) (width 0.2) (layer "B.Cu") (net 3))
 (segment (start 139.599999 95.852842) (end 139.599999 109.400001) (width 0.2) (layer "B.Cu") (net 3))
 (segment (start 167.599999 135.852842) (end 189.147158 135.852842) (width 0.2) (layer "B.Cu") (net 1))
 (segment (start 195.600001 129.399999) (end 195.600001 95.647158) (width 0.2) (layer "B.Cu") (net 1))
 (segment (start 189.147158 135.852842) (end 195.600001 129.399999) (width 0.2) (layer "B.Cu") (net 1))
 (segment (start 174 62.103) (end 174 56) (width 0.2) (layer "B.Cu") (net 13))
 (segment (start 177.835 65.938) (end 174 62.103) (width 0.2) (layer "B.Cu") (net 13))
 (segment (start 169 63) (end 168 63) (width 0.2) (layer "F.Cu") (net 7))
 (segment (start 170 64) (end 169 63) (width 0.2) (layer "F.Cu") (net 7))
 (via (at 168 63) (size 0.6) (drill 0.3) (layers "F.Cu" "B.Cu") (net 7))
 (via (at 170 64) (size 0.6) (drill 0.3) (layers "F.Cu" "B.Cu") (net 7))
 (segment (start 180 74) (end 170 64) (width 0.2) (layer "B.Cu") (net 7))
 (segment (start 164.27 62.19) (end 140 62.19) (width 0.2) (layer "B.Cu") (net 7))
 (segment (start 168 61.54) (end 166.46 60) (width 0.2) (layer "B.Cu") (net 7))
 (segment (start 180 75) (end 180 74) (width 0.2) (layer "B.Cu") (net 7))
 (segment (start 194 66) (end 193.962942 66) (width 0.2) (layer "B.Cu") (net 7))
 (segment (start 166.46 60) (end 164.27 62.19) (width 0.2) (layer "B.Cu") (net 7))
 (segment (start 194 65.938) (end 194 66) (width 0.2) (layer "B.Cu") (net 7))
 (segment (start 193.962942 66) (end 184.962942 75) (width 0.2) (layer "B.Cu") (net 7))
 (segment (start 184.962942 75) (end 180 75) (width 0.2) (layer "B.Cu") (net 7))
 (segment (start 168 63) (end 168 61.54) (width 0.2) (layer "B.Cu") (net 7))
 (segment (start 164.27 64.73) (end 140 64.73) (width 0.2) (layer "F.Cu") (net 8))
 (segment (start 169 60) (end 164.27 64.73) (width 0.2) (layer "F.Cu") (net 8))
 (segment (start 195.676 65.074) (end 195.676 69.317058) (width 0.2) (layer "B.Cu") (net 8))
 (segment (start 185.949 75.949) (end 179.759936 75.949) (width 0.2) (layer "B.Cu") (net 8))
 (segment (start 186 76) (end 185.949 75.949) (width 0.2) (layer "B.Cu") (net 8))
 (segment (start 179.759936 75.949) (end 169 65.189064) (width 0.2) (layer "B.Cu") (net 8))
 (segment (start 169 65.189064) (end 169 60) (width 0.2) (layer "B.Cu") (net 8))
 (segment (start 194 63.398) (end 195.676 65.074) (width 0.2) (layer "B.Cu") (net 8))
 (segment (start 188.993058 76) (end 186 76) (width 0.2) (layer "B.Cu") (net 8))
 (segment (start 195.676 69.317058) (end 188.993058 76) (width 0.2) (layer "B.Cu") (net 8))
 (segment (start 163.92 62.92) (end 164 63) (width 0.2) (layer "F.Cu") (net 2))
 (segment (start 172 58) (end 163 58) (width 0.2) (layer "F.Cu") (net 2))
 (segment (start 163.92 60) (end 163 59.08) (width 0.2) (layer "F.Cu") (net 2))
 (segment (start 139.35 59) (end 137 59) (width 0.2) (layer "F.Cu") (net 2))
 (segment (start 163.92 60) (end 163.92 62.92) (width 0.2) (layer "F.Cu") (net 2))
 (segment (start 175.182765 54.817235) (end 172 58) (width 0.2) (layer "F.Cu") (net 2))
 (segment (start 163 59.08) (end 163 58) (width 0.2) (layer "F.Cu") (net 2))
 (segment (start 140 59.65) (end 139.35 59) (width 0.2) (layer "F.Cu") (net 2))
 (via (at 164 63) (size 0.6) (drill 0.3) (layers "F.Cu" "B.Cu") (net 2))
 (via (at 163 58) (size 0.6) (drill 0.3) (layers "F.Cu" "B.Cu") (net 2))
 (via (at 137 59) (size 0.6) (drill 0.3) (layers "F.Cu" "B.Cu") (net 2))
 (via (at 175.182765 54.817235) (size 0.6) (drill 0.3) (layers "F.Cu" "B.Cu") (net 2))
 (segment (start 139.599999 94.352842) (end 139.599999 92.117759) (width 0.2) (layer "B.Cu") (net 2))
 (segment (start 148.38 102.38) (end 148.38 114.92) (width 0.2) (layer "B.Cu") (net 2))
 (segment (start 167.599999 115.079999) (end 167.44 114.92) (width 0.2) (layer "B.Cu") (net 2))
 (segment (start 163 58) (end 162.400001 57.400001) (width 0.2) (layer "B.Cu") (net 2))
 (segment (start 167.599999 134.352842) (end 167.599999 115.079999) (width 0.2) (layer "B.Cu") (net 2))
 (segment (start 162.400001 57.400001) (end 142.249999 57.400001) (width 0.2) (layer "B.Cu") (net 2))
 (segment (start 176.14353 55.778) (end 175.182765 54.817235) (width 0.2) (layer "B.Cu") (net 2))
 (segment (start 139.599999 92.117759) (end 139.48224 92) (width 0.2) (layer "B.Cu") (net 2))
 (segment (start 135 92) (end 135 58.775) (width 0.2) (layer "B.Cu") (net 2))
 (segment (start 167.44 114.92) (end 148.38 114.92) (width 0.2) (layer "B.Cu") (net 2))
 (segment (start 139.48224 92) (end 135 92) (width 0.2) (layer "B.Cu") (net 2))
 (segment (start 139.599999 94.352842) (end 140.352842 94.352842) (width 0.2) (layer "B.Cu") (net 2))
 (segment (start 162.400001 57.400001) (end 162.400001 55.96) (width 0.2) (layer "B.Cu") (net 2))
 (segment (start 177.835 55.778) (end 176.14353 55.778) (width 0.2) (layer "B.Cu") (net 2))
 (segment (start 140.352842 94.352842) (end 148.38 102.38) (width 0.2) (layer "B.Cu") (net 2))
 (segment (start 142.249999 57.400001) (end 140 59.65) (width 0.2) (layer "B.Cu") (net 2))
 (segment (start 136.775 58.775) (end 135 58.775) (width 0.2) (layer "B.Cu") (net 2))
 (segment (start 186.49 114.92) (end 167.44 114.92) (width 0.2) (layer "B.Cu") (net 2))
 (segment (start 191.45 109.96) (end 186.49 114.92) (width 0.2) (layer "B.Cu") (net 2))
 (segment (start 190.400001 102.950001) (end 190.400001 95.647158) (width 0.2) (layer "B.Cu") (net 2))
 (segment (start 137 59) (end 136.775 58.775) (width 0.2) (layer "B.Cu") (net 2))
 (segment (start 191.45 104) (end 191.45 109.96) (width 0.2) (layer "B.Cu") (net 2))
 (segment (start 191.45 104) (end 190.400001 102.950001) (width 0.2) (layer "B.Cu") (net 2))
 (segment (start 164 63) (end 164 64) (width 0.2) (layer "B.Cu") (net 2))
 (segment (start 151 109) (end 150.49 109) (width 0.2) (layer "F.Cu") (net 5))
 (segment (start 150.49 109) (end 142.03 117.46) (width 0.2) (layer "F.Cu") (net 5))
 (via (at 151 109) (size 0.6) (drill 0.3) (layers "F.Cu" "B.Cu") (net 5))
 (segment (start 196.879 56.117) (end 196.879 78.538043) (width 0.2) (layer "B.Cu") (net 5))
 (segment (start 194 53.238) (end 196.879 56.117) (width 0.2) (layer "B.Cu") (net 5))
 (segment (start 196.879 78.538043) (end 166.417043 109) (width 0.2) (layer "B.Cu") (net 5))
 (segment (start 166.417043 109) (end 151 109) (width 0.2) (layer "B.Cu") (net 5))
 (segment (start 161 104) (end 161.09 104.09) (width 0.2) (layer "F.Cu") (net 9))
 (segment (start 161.09 104.09) (end 161.09 117.46) (width 0.2) (layer "F.Cu") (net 9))
 (segment (start 161 103) (end 161 104) (width 0.2) (layer "F.Cu") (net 9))
 (via (at 161 103) (size 0.6) (drill 0.3) (layers "F.Cu" "B.Cu") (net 9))
 (segment (start 196.478 58.256) (end 196.478 78.371943) (width 0.2) (layer "B.Cu") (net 9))
 (segment (start 171.849943 103) (end 161 103) (width 0.2) (layer "B.Cu") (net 9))
 (segment (start 194 55.778) (end 196.478 58.256) (width 0.2) (layer "B.Cu") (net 9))
 (segment (start 196.478 78.371943) (end 171.849943 103) (width 0.2) (layer "B.Cu") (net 9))
 (segment (start 180.14 94.86) (end 180.14 117.46) (width 0.2) (layer "F.Cu") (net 6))
 (segment (start 181 93) (end 181 94) (width 0.2) (layer "F.Cu") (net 6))
 (segment (start 181 94) (end 180.14 94.86) (width 0.2) (layer "F.Cu") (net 6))
 (via (at 181 93) (size 0.6) (drill 0.3) (layers "F.Cu" "B.Cu") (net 6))
 (segment (start 194 58.318) (end 196.077 60.395) (width 0.2) (layer "B.Cu") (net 6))
 (segment (start 196.077 60.395) (end 196.077 77.923) (width 0.2) (layer "B.Cu") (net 6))
 (segment (start 196.077 77.923) (end 181 93) (width 0.2) (layer "B.Cu") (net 6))
 (segment (start 134 58) (end 134 92) (width 0.2) (layer "F.Cu") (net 4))
 (segment (start 161.38 60) (end 161.38 62.38) (width 0.2) (layer "F.Cu") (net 4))
 (segment (start 161.38 60) (end 142.89 60) (width 0.2) (layer "F.Cu") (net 4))
 (segment (start 194 104) (end 197 104) (width 0.2) (layer "F.Cu") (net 4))
 (segment (start 194 104) (end 194 113.33153) (width 0.2) (layer "F.Cu") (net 4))
 (segment (start 142.89 60) (end 140 57.11) (width 0.2) (layer "F.Cu") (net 4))
 (segment (start 194 113.33153) (end 168.33153 139) (width 0.2) (layer "F.Cu") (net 4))
 (segment (start 140 57.11) (end 134.89 57.11) (width 0.2) (layer "F.Cu") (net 4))
 (segment (start 168.33153 139) (end 166 139) (width 0.2) (layer "F.Cu") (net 4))
 (segment (start 161.38 62.38) (end 162 63) (width 0.2) (layer "F.Cu") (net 4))
 (segment (start 134 92) (end 132 94) (width 0.2) (layer "F.Cu") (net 4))
 (segment (start 161.38 60) (end 162 59.38) (width 0.2) (layer "F.Cu") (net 4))
 (segment (start 134.89 57.11) (end 134 58) (width 0.2) (layer "F.Cu") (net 4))
 (segment (start 162 59.38) (end 162 53) (width 0.2) (layer "F.Cu") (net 4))
 (via (at 132 94) (size 0.6) (drill 0.3) (layers "F.Cu" "B.Cu") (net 4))
 (via (at 134 58) (size 0.6) (drill 0.3) (layers "F.Cu" "B.Cu") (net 4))
 (via (at 166 139) (size 0.6) (drill 0.3) (layers "F.Cu" "B.Cu") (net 4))
 (via (at 162 53) (size 0.6) (drill 0.3) (layers "F.Cu" "B.Cu") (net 4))
 (via (at 194 104) (size 0.6) (drill 0.3) (layers "F.Cu" "B.Cu") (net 4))
 (via (at 162 63) (size 0.6) (drill 0.3) (layers "F.Cu" "B.Cu") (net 4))
 (via (at 197 104) (size 0.6) (drill 0.3) (layers "F.Cu" "B.Cu") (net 4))
 (segment (start 134.775 57.225) (end 134 58) (width 0.2) (layer "B.Cu") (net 4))
 (segment (start 166 52) (end 163 52) (width 0.2) (layer "B.Cu") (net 4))
 (segment (start 160 135.852842) (end 162.399999 135.852842) (width 0.2) (layer "B.Cu") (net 4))
 (segment (start 195.600001 94.147158) (end 195.689915 94.147158) (width 0.2) (layer "B.Cu") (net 4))
 (segment (start 180 76.65) (end 175.1 76.65) (width 0.2) (layer "B.Cu") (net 4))
 (segment (start 177.835 58.318) (end 173.977 54.46) (width 0.2) (layer "B.Cu") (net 4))
 (segment (start 177.835 58.165) (end 178 58) (width 0.2) (layer "B.Cu") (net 4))
 (segment (start 167.600001 53.600001) (end 166 52) (width 0.2) (layer "B.Cu") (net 4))
 (segment (start 167.600001 54.46) (end 167.600001 53.600001) (width 0.2) (layer "B.Cu") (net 4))
 (segment (start 195.689915 94.147158) (end 197 95.457243) (width 0.2) (layer "B.Cu") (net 4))
 (segment (start 163 52) (end 162 53) (width 0.2) (layer "B.Cu") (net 4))
 (segment (start 186 77.65) (end 181 77.65) (width 0.2) (layer "B.Cu") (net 4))
 (segment (start 134.399999 95.852842) (end 134.399999 133.967099) (width 0.2) (layer "B.Cu") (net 4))
 (segment (start 133.852842 95.852842) (end 134.399999 95.852842) (width 0.2) (layer "B.Cu") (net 4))
 (segment (start 175.1 76.65) (end 162.45 64) (width 0.2) (layer "B.Cu") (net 4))
 (segment (start 132 94) (end 133.852842 95.852842) (width 0.2) (layer "B.Cu") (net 4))
 (segment (start 162 63) (end 162 63.55) (width 0.2) (layer "B.Cu") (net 4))
 (segment (start 162 63.55) (end 162.45 64) (width 0.2) (layer "B.Cu") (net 4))
 (segment (start 134.399999 133.967099) (end 136.285742 135.852842) (width 0.2) (layer "B.Cu") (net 4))
 (segment (start 193 104) (end 194 104) (width 0.2) (layer "B.Cu") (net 4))
 (segment (start 166 139) (end 163.147158 139) (width 0.2) (layer "B.Cu") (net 4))
 (segment (start 173.977 54.46) (end 167.600001 54.46) (width 0.2) (layer "B.Cu") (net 4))
 (segment (start 181 77.65) (end 180 76.65) (width 0.2) (layer "B.Cu") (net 4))
 (segment (start 197 95.457243) (end 197 104) (width 0.2) (layer "B.Cu") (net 4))
 (segment (start 163.147158 139) (end 160 135.852842) (width 0.2) (layer "B.Cu") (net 4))
 (segment (start 136.285742 135.852842) (end 160 135.852842) (width 0.2) (layer "B.Cu") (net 4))
 (segment (start 135 57.225) (end 134.775 57.225) (width 0.2) (layer "B.Cu") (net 4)))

